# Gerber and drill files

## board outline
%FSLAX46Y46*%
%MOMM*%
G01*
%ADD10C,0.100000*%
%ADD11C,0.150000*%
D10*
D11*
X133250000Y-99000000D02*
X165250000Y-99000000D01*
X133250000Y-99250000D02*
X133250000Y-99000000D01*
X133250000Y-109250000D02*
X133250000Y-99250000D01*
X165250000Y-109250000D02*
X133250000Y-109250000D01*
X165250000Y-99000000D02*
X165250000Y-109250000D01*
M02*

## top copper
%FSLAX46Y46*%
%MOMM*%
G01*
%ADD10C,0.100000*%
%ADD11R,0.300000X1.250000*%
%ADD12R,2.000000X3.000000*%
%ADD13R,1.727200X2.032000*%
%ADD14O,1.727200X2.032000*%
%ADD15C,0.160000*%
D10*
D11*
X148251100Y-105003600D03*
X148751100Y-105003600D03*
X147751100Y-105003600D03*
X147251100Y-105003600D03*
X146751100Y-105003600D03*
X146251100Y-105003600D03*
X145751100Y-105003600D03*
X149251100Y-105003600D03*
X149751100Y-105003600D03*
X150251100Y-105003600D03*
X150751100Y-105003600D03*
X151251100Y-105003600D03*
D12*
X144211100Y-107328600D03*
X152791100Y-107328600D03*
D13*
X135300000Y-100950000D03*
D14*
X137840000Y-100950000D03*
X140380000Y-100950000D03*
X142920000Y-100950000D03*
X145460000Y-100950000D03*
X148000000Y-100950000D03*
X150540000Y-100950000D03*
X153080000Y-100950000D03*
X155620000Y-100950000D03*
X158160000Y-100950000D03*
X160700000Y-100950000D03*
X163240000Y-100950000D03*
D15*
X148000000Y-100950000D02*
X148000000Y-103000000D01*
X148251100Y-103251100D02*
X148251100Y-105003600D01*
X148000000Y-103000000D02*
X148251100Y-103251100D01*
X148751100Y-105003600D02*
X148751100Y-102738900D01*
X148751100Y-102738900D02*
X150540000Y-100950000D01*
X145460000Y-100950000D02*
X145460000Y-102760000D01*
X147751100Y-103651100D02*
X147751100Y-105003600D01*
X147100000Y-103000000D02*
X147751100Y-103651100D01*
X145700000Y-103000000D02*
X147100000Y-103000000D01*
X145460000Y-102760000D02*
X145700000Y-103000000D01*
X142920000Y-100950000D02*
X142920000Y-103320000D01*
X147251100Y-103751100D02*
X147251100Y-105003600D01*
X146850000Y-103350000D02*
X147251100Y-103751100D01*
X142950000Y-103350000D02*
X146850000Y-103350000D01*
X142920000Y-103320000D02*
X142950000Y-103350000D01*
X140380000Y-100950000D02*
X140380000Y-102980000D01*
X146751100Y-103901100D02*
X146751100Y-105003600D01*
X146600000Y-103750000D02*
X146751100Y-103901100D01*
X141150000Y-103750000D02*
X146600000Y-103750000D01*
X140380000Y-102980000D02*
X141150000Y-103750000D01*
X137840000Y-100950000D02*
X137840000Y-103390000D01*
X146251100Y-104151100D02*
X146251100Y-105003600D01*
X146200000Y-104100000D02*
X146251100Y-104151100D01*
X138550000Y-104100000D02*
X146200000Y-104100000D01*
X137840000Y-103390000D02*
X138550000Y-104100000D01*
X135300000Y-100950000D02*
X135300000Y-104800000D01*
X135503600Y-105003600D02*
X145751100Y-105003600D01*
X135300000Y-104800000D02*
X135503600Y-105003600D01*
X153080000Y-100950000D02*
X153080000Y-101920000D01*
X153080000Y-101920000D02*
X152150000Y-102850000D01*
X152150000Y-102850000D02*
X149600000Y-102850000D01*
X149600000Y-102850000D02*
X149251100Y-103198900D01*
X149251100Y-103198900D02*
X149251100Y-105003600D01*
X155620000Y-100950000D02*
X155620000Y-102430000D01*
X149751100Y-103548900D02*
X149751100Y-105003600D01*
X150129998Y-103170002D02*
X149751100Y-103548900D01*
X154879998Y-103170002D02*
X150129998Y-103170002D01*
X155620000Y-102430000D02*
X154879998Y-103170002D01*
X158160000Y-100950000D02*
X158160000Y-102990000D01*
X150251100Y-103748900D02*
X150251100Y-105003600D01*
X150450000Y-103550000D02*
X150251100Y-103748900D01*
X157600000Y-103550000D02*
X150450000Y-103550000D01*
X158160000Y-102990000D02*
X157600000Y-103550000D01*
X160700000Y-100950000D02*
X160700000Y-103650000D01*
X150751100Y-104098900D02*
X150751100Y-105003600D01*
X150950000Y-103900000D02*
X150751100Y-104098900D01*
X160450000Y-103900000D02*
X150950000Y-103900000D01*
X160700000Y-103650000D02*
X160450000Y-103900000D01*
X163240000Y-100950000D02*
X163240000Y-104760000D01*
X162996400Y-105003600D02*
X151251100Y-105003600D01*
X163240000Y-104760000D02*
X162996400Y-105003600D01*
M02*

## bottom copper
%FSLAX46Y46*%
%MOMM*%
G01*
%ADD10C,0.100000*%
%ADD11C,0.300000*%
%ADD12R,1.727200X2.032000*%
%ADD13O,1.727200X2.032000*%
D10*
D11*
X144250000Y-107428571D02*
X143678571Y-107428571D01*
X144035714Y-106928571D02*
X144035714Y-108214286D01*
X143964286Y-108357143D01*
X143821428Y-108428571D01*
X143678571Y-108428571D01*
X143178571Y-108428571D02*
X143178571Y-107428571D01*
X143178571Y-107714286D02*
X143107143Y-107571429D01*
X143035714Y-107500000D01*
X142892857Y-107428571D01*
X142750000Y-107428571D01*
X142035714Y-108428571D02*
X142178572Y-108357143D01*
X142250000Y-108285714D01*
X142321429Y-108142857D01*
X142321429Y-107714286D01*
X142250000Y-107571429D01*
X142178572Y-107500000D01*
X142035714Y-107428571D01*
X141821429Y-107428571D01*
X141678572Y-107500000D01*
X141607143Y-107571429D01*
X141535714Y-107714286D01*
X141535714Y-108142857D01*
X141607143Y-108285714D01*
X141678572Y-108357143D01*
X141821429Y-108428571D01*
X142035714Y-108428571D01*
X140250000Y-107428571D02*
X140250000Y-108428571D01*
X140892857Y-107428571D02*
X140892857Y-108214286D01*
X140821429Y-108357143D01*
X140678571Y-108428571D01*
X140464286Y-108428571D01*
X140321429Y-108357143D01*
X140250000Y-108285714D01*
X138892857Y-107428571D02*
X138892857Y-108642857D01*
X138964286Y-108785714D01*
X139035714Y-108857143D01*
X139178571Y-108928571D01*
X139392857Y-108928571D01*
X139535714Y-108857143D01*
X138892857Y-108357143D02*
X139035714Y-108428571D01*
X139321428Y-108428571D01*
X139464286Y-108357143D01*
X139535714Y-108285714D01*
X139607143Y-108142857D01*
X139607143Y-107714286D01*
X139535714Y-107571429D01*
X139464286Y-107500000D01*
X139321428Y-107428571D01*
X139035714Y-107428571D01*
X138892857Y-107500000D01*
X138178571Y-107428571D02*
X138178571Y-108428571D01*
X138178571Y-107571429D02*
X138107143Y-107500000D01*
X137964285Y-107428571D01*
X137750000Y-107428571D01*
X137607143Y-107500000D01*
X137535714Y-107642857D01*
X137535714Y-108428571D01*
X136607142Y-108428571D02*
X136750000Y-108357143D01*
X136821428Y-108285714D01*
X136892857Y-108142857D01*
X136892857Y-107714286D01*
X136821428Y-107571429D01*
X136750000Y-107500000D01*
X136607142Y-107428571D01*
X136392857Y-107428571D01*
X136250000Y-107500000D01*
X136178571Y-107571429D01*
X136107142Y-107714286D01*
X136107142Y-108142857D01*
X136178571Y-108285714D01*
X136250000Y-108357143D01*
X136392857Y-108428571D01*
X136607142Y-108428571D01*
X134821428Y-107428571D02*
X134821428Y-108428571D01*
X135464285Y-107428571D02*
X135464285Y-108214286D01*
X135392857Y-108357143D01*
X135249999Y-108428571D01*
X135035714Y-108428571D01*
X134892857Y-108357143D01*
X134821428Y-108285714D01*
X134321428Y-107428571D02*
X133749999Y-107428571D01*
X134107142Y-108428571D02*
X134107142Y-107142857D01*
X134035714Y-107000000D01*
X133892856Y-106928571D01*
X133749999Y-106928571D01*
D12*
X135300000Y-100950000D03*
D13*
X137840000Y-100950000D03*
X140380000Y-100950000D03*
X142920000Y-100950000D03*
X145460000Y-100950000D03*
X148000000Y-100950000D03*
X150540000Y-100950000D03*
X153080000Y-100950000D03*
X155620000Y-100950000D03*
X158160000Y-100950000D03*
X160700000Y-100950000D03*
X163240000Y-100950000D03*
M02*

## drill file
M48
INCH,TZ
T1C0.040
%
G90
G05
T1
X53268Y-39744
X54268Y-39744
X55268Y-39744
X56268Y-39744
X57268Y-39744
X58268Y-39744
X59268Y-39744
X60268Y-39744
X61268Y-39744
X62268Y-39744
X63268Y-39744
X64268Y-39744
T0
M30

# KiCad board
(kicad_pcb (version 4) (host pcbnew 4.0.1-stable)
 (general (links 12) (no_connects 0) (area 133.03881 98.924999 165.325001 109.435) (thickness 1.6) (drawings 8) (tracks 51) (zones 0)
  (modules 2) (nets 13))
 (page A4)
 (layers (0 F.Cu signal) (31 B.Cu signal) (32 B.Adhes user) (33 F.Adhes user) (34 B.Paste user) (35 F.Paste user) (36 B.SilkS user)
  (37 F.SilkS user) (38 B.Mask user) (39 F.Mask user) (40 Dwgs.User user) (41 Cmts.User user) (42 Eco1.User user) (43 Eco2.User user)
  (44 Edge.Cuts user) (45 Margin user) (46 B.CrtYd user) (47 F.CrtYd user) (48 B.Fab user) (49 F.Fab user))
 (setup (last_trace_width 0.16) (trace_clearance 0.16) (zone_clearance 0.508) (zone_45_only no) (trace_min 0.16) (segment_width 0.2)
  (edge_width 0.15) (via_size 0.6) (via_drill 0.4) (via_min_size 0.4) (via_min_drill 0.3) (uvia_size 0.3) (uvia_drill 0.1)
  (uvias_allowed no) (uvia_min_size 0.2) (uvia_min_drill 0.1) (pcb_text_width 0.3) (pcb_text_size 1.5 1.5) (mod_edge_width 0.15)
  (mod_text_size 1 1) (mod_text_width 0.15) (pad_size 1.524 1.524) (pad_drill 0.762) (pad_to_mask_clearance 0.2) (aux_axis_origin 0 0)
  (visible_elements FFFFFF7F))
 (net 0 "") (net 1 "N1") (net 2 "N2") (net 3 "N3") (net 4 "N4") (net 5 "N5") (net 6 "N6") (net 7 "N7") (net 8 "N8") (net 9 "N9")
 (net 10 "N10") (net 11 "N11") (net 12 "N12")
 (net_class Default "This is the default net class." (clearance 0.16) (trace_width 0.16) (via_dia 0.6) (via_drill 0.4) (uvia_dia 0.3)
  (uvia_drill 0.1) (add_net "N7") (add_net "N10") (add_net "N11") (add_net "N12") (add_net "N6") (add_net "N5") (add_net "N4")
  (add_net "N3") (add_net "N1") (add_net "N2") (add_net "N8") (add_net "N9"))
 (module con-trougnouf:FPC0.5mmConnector (layer F.Cu) (at 148.5011 105.0036)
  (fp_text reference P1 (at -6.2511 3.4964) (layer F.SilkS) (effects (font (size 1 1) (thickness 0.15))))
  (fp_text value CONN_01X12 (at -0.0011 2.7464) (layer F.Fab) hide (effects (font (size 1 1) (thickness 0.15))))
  (pad 6 smd rect (at -0.25 0) (size 0.3 1.25) (layers F.Cu F.Paste F.Mask) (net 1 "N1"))
  (pad 7 smd rect (at 0.25 0) (size 0.3 1.25) (layers F.Cu F.Paste F.Mask) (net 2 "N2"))
  (pad 5 smd rect (at -0.75 0) (size 0.3 1.25) (layers F.Cu F.Paste F.Mask) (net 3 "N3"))
  (pad 4 smd rect (at -1.25 0) (size 0.3 1.25) (layers F.Cu F.Paste F.Mask) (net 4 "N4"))
  (pad 3 smd rect (at -1.75 0) (size 0.3 1.25) (layers F.Cu F.Paste F.Mask) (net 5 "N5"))
  (pad 2 smd rect (at -2.25 0) (size 0.3 1.25) (layers F.Cu F.Paste F.Mask) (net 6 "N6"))
  (pad 1 smd rect (at -2.75 0) (size 0.3 1.25) (layers F.Cu F.Paste F.Mask) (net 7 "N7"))
  (pad 8 smd rect (at 0.75 0) (size 0.3 1.25) (layers F.Cu F.Paste F.Mask) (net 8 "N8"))
  (pad 9 smd rect (at 1.25 0) (size 0.3 1.25) (layers F.Cu F.Paste F.Mask) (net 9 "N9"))
  (pad 10 smd rect (at 1.75 0) (size 0.3 1.25) (layers F.Cu F.Paste F.Mask) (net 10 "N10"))
  (pad 11 smd rect (at 2.25 0) (size 0.3 1.25) (layers F.Cu F.Paste F.Mask) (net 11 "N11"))
  (pad 12 smd rect (at 2.75 0) (size 0.3 1.25) (layers F.Cu F.Paste F.Mask) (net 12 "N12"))
  (pad "" smd rect (at -4.29 2.325) (size 2 3) (layers F.Cu F.Paste F.Mask))
  (pad "" smd rect (at 4.29 2.325) (size 2 3) (layers F.Cu F.Paste F.Mask)))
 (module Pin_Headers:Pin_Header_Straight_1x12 (layer F.Cu) (at 135.3 100.95 90)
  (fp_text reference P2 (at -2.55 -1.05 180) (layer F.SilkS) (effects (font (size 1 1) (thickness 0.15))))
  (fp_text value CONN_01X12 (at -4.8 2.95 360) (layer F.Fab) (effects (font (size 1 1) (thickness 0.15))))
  (pad 1 thru_hole rect (at 0 0 90) (size 2.032 1.7272) (drill 1.016) (layers *.Cu *.Mask F.SilkS) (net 7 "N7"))
  (pad 2 thru_hole oval (at 0 2.54 90) (size 2.032 1.7272) (drill 1.016) (layers *.Cu *.Mask F.SilkS) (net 6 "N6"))
  (pad 3 thru_hole oval (at 0 5.08 90) (size 2.032 1.7272) (drill 1.016) (layers *.Cu *.Mask F.SilkS) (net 5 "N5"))
  (pad 4 thru_hole oval (at 0 7.62 90) (size 2.032 1.7272) (drill 1.016) (layers *.Cu *.Mask F.SilkS) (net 4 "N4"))
  (pad 5 thru_hole oval (at 0 10.16 90) (size 2.032 1.7272) (drill 1.016) (layers *.Cu *.Mask F.SilkS) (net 3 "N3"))
  (pad 6 thru_hole oval (at 0 12.7 90) (size 2.032 1.7272) (drill 1.016) (layers *.Cu *.Mask F.SilkS) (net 1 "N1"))
  (pad 7 thru_hole oval (at 0 15.24 90) (size 2.032 1.7272) (drill 1.016) (layers *.Cu *.Mask F.SilkS) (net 2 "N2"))
  (pad 8 thru_hole oval (at 0 17.78 90) (size 2.032 1.7272) (drill 1.016) (layers *.Cu *.Mask F.SilkS) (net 8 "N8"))
  (pad 9 thru_hole oval (at 0 20.32 90) (size 2.032 1.7272) (drill 1.016) (layers *.Cu *.Mask F.SilkS) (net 9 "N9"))
  (pad 10 thru_hole oval (at 0 22.86 90) (size 2.032 1.7272) (drill 1.016) (layers *.Cu *.Mask F.SilkS) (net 10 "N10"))
  (pad 11 thru_hole oval (at 0 25.4 90) (size 2.032 1.7272) (drill 1.016) (layers *.Cu *.Mask F.SilkS) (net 11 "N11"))
  (pad 12 thru_hole oval (at 0 27.94 90) (size 2.032 1.7272) (drill 1.016) (layers *.Cu *.Mask F.SilkS) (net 12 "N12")))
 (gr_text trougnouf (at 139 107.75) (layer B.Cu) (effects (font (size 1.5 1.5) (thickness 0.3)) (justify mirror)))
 (gr_line (start 133.25 99) (end 165.25 99) (angle 90) (layer Edge.Cuts) (width 0.15))
 (gr_line (start 133.25 99.25) (end 133.25 99) (angle 90) (layer Edge.Cuts) (width 0.15))
 (gr_line (start 133.25 109.25) (end 133.25 99.25) (angle 90) (layer Edge.Cuts) (width 0.15))
 (gr_line (start 165.25 109.25) (end 133.25 109.25) (angle 90) (layer Edge.Cuts) (width 0.15))
 (gr_line (start 165.25 99) (end 165.25 109.25) (angle 90) (layer Edge.Cuts) (width 0.15))
 (segment (start 148 100.95) (end 148 103) (width 0.16) (layer F.Cu) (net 1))
 (segment (start 148.2511 103.2511) (end 148.2511 105.0036) (width 0.16) (layer F.Cu) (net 1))
 (segment (start 148 103) (end 148.2511 103.2511) (width 0.16) (layer F.Cu) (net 1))
 (segment (start 148.7511 105.0036) (end 148.7511 102.7389) (width 0.16) (layer F.Cu) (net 2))
 (segment (start 148.7511 102.7389) (end 150.54 100.95) (width 0.16) (layer F.Cu) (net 2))
 (segment (start 145.46 100.95) (end 145.46 102.76) (width 0.16) (layer F.Cu) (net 3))
 (segment (start 147.7511 103.6511) (end 147.7511 105.0036) (width 0.16) (layer F.Cu) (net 3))
 (segment (start 147.1 103) (end 147.7511 103.6511) (width 0.16) (layer F.Cu) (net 3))
 (segment (start 145.7 103) (end 147.1 103) (width 0.16) (layer F.Cu) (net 3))
 (segment (start 145.46 102.76) (end 145.7 103) (width 0.16) (layer F.Cu) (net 3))
 (segment (start 142.92 100.95) (end 142.92 103.32) (width 0.16) (layer F.Cu) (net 4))
 (segment (start 147.2511 103.7511) (end 147.2511 105.0036) (width 0.16) (layer F.Cu) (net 4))
 (segment (start 146.85 103.35) (end 147.2511 103.7511) (width 0.16) (layer F.Cu) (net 4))
 (segment (start 142.95 103.35) (end 146.85 103.35) (width 0.16) (layer F.Cu) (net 4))
 (segment (start 142.92 103.32) (end 142.95 103.35) (width 0.16) (layer F.Cu) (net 4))
 (segment (start 140.38 100.95) (end 140.38 102.98) (width 0.16) (layer F.Cu) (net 5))
 (segment (start 146.7511 103.9011) (end 146.7511 105.0036) (width 0.16) (layer F.Cu) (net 5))
 (segment (start 146.6 103.75) (end 146.7511 103.9011) (width 0.16) (layer F.Cu) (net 5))
 (segment (start 141.15 103.75) (end 146.6 103.75) (width 0.16) (layer F.Cu) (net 5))
 (segment (start 140.38 102.98) (end 141.15 103.75) (width 0.16) (layer F.Cu) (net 5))
 (segment (start 137.84 100.95) (end 137.84 103.39) (width 0.16) (layer F.Cu) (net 6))
 (segment (start 146.2511 104.1511) (end 146.2511 105.0036) (width 0.16) (layer F.Cu) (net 6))
 (segment (start 146.2 104.1) (end 146.2511 104.1511) (width 0.16) (layer F.Cu) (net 6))
 (segment (start 138.55 104.1) (end 146.2 104.1) (width 0.16) (layer F.Cu) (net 6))
 (segment (start 137.84 103.39) (end 138.55 104.1) (width 0.16) (layer F.Cu) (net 6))
 (segment (start 135.3 100.95) (end 135.3 104.8) (width 0.16) (layer F.Cu) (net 7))
 (segment (start 135.5036 105.0036) (end 145.7511 105.0036) (width 0.16) (layer F.Cu) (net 7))
 (segment (start 135.3 104.8) (end 135.5036 105.0036) (width 0.16) (layer F.Cu) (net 7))
 (segment (start 153.08 100.95) (end 153.08 101.92) (width 0.16) (layer F.Cu) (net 8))
 (segment (start 153.08 101.92) (end 152.15 102.85) (width 0.16) (layer F.Cu) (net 8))
 (segment (start 152.15 102.85) (end 149.6 102.85) (width 0.16) (layer F.Cu) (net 8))
 (segment (start 149.6 102.85) (end 149.2511 103.1989) (width 0.16) (layer F.Cu) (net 8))
 (segment (start 149.2511 103.1989) (end 149.2511 105.0036) (width 0.16) (layer F.Cu) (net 8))
 (segment (start 155.62 100.95) (end 155.62 102.43) (width 0.16) (layer F.Cu) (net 9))
 (segment (start 149.7511 103.5489) (end 149.7511 105.0036) (width 0.16) (layer F.Cu) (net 9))
 (segment (start 150.129998 103.170002) (end 149.7511 103.5489) (width 0.16) (layer F.Cu) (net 9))
 (segment (start 154.879998 103.170002) (end 150.129998 103.170002) (width 0.16) (layer F.Cu) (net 9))
 (segment (start 155.62 102.43) (end 154.879998 103.170002) (width 0.16) (layer F.Cu) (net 9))
 (segment (start 158.16 100.95) (end 158.16 102.99) (width 0.16) (layer F.Cu) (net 10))
 (segment (start 150.2511 103.7489) (end 150.2511 105.0036) (width 0.16) (layer F.Cu) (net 10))
 (segment (start 150.45 103.55) (end 150.2511 103.7489) (width 0.16) (layer F.Cu) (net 10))
 (segment (start 157.6 103.55) (end 150.45 103.55) (width 0.16) (layer F.Cu) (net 10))
 (segment (start 158.16 102.99) (end 157.6 103.55) (width 0.16) (layer F.Cu) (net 10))
 (segment (start 160.7 100.95) (end 160.7 103.65) (width 0.16) (layer F.Cu) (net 11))
 (segment (start 150.7511 104.0989) (end 150.7511 105.0036) (width 0.16) (layer F.Cu) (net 11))
 (segment (start 150.95 103.9) (end 150.7511 104.0989) (width 0.16) (layer F.Cu) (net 11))
 (segment (start 160.45 103.9) (end 150.95 103.9) (width 0.16) (layer F.Cu) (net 11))
 (segment (start 160.7 103.65) (end 160.45 103.9) (width 0.16) (layer F.Cu) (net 11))
 (segment (start 163.24 100.95) (end 163.24 104.76) (width 0.16) (layer F.Cu) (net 12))
 (segment (start 162.9964 105.0036) (end 151.2511 105.0036) (width 0.16) (layer F.Cu) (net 12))
 (segment (start 163.24 104.76) (end 162.9964 105.0036) (width 0.16) (layer F.Cu) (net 12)))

